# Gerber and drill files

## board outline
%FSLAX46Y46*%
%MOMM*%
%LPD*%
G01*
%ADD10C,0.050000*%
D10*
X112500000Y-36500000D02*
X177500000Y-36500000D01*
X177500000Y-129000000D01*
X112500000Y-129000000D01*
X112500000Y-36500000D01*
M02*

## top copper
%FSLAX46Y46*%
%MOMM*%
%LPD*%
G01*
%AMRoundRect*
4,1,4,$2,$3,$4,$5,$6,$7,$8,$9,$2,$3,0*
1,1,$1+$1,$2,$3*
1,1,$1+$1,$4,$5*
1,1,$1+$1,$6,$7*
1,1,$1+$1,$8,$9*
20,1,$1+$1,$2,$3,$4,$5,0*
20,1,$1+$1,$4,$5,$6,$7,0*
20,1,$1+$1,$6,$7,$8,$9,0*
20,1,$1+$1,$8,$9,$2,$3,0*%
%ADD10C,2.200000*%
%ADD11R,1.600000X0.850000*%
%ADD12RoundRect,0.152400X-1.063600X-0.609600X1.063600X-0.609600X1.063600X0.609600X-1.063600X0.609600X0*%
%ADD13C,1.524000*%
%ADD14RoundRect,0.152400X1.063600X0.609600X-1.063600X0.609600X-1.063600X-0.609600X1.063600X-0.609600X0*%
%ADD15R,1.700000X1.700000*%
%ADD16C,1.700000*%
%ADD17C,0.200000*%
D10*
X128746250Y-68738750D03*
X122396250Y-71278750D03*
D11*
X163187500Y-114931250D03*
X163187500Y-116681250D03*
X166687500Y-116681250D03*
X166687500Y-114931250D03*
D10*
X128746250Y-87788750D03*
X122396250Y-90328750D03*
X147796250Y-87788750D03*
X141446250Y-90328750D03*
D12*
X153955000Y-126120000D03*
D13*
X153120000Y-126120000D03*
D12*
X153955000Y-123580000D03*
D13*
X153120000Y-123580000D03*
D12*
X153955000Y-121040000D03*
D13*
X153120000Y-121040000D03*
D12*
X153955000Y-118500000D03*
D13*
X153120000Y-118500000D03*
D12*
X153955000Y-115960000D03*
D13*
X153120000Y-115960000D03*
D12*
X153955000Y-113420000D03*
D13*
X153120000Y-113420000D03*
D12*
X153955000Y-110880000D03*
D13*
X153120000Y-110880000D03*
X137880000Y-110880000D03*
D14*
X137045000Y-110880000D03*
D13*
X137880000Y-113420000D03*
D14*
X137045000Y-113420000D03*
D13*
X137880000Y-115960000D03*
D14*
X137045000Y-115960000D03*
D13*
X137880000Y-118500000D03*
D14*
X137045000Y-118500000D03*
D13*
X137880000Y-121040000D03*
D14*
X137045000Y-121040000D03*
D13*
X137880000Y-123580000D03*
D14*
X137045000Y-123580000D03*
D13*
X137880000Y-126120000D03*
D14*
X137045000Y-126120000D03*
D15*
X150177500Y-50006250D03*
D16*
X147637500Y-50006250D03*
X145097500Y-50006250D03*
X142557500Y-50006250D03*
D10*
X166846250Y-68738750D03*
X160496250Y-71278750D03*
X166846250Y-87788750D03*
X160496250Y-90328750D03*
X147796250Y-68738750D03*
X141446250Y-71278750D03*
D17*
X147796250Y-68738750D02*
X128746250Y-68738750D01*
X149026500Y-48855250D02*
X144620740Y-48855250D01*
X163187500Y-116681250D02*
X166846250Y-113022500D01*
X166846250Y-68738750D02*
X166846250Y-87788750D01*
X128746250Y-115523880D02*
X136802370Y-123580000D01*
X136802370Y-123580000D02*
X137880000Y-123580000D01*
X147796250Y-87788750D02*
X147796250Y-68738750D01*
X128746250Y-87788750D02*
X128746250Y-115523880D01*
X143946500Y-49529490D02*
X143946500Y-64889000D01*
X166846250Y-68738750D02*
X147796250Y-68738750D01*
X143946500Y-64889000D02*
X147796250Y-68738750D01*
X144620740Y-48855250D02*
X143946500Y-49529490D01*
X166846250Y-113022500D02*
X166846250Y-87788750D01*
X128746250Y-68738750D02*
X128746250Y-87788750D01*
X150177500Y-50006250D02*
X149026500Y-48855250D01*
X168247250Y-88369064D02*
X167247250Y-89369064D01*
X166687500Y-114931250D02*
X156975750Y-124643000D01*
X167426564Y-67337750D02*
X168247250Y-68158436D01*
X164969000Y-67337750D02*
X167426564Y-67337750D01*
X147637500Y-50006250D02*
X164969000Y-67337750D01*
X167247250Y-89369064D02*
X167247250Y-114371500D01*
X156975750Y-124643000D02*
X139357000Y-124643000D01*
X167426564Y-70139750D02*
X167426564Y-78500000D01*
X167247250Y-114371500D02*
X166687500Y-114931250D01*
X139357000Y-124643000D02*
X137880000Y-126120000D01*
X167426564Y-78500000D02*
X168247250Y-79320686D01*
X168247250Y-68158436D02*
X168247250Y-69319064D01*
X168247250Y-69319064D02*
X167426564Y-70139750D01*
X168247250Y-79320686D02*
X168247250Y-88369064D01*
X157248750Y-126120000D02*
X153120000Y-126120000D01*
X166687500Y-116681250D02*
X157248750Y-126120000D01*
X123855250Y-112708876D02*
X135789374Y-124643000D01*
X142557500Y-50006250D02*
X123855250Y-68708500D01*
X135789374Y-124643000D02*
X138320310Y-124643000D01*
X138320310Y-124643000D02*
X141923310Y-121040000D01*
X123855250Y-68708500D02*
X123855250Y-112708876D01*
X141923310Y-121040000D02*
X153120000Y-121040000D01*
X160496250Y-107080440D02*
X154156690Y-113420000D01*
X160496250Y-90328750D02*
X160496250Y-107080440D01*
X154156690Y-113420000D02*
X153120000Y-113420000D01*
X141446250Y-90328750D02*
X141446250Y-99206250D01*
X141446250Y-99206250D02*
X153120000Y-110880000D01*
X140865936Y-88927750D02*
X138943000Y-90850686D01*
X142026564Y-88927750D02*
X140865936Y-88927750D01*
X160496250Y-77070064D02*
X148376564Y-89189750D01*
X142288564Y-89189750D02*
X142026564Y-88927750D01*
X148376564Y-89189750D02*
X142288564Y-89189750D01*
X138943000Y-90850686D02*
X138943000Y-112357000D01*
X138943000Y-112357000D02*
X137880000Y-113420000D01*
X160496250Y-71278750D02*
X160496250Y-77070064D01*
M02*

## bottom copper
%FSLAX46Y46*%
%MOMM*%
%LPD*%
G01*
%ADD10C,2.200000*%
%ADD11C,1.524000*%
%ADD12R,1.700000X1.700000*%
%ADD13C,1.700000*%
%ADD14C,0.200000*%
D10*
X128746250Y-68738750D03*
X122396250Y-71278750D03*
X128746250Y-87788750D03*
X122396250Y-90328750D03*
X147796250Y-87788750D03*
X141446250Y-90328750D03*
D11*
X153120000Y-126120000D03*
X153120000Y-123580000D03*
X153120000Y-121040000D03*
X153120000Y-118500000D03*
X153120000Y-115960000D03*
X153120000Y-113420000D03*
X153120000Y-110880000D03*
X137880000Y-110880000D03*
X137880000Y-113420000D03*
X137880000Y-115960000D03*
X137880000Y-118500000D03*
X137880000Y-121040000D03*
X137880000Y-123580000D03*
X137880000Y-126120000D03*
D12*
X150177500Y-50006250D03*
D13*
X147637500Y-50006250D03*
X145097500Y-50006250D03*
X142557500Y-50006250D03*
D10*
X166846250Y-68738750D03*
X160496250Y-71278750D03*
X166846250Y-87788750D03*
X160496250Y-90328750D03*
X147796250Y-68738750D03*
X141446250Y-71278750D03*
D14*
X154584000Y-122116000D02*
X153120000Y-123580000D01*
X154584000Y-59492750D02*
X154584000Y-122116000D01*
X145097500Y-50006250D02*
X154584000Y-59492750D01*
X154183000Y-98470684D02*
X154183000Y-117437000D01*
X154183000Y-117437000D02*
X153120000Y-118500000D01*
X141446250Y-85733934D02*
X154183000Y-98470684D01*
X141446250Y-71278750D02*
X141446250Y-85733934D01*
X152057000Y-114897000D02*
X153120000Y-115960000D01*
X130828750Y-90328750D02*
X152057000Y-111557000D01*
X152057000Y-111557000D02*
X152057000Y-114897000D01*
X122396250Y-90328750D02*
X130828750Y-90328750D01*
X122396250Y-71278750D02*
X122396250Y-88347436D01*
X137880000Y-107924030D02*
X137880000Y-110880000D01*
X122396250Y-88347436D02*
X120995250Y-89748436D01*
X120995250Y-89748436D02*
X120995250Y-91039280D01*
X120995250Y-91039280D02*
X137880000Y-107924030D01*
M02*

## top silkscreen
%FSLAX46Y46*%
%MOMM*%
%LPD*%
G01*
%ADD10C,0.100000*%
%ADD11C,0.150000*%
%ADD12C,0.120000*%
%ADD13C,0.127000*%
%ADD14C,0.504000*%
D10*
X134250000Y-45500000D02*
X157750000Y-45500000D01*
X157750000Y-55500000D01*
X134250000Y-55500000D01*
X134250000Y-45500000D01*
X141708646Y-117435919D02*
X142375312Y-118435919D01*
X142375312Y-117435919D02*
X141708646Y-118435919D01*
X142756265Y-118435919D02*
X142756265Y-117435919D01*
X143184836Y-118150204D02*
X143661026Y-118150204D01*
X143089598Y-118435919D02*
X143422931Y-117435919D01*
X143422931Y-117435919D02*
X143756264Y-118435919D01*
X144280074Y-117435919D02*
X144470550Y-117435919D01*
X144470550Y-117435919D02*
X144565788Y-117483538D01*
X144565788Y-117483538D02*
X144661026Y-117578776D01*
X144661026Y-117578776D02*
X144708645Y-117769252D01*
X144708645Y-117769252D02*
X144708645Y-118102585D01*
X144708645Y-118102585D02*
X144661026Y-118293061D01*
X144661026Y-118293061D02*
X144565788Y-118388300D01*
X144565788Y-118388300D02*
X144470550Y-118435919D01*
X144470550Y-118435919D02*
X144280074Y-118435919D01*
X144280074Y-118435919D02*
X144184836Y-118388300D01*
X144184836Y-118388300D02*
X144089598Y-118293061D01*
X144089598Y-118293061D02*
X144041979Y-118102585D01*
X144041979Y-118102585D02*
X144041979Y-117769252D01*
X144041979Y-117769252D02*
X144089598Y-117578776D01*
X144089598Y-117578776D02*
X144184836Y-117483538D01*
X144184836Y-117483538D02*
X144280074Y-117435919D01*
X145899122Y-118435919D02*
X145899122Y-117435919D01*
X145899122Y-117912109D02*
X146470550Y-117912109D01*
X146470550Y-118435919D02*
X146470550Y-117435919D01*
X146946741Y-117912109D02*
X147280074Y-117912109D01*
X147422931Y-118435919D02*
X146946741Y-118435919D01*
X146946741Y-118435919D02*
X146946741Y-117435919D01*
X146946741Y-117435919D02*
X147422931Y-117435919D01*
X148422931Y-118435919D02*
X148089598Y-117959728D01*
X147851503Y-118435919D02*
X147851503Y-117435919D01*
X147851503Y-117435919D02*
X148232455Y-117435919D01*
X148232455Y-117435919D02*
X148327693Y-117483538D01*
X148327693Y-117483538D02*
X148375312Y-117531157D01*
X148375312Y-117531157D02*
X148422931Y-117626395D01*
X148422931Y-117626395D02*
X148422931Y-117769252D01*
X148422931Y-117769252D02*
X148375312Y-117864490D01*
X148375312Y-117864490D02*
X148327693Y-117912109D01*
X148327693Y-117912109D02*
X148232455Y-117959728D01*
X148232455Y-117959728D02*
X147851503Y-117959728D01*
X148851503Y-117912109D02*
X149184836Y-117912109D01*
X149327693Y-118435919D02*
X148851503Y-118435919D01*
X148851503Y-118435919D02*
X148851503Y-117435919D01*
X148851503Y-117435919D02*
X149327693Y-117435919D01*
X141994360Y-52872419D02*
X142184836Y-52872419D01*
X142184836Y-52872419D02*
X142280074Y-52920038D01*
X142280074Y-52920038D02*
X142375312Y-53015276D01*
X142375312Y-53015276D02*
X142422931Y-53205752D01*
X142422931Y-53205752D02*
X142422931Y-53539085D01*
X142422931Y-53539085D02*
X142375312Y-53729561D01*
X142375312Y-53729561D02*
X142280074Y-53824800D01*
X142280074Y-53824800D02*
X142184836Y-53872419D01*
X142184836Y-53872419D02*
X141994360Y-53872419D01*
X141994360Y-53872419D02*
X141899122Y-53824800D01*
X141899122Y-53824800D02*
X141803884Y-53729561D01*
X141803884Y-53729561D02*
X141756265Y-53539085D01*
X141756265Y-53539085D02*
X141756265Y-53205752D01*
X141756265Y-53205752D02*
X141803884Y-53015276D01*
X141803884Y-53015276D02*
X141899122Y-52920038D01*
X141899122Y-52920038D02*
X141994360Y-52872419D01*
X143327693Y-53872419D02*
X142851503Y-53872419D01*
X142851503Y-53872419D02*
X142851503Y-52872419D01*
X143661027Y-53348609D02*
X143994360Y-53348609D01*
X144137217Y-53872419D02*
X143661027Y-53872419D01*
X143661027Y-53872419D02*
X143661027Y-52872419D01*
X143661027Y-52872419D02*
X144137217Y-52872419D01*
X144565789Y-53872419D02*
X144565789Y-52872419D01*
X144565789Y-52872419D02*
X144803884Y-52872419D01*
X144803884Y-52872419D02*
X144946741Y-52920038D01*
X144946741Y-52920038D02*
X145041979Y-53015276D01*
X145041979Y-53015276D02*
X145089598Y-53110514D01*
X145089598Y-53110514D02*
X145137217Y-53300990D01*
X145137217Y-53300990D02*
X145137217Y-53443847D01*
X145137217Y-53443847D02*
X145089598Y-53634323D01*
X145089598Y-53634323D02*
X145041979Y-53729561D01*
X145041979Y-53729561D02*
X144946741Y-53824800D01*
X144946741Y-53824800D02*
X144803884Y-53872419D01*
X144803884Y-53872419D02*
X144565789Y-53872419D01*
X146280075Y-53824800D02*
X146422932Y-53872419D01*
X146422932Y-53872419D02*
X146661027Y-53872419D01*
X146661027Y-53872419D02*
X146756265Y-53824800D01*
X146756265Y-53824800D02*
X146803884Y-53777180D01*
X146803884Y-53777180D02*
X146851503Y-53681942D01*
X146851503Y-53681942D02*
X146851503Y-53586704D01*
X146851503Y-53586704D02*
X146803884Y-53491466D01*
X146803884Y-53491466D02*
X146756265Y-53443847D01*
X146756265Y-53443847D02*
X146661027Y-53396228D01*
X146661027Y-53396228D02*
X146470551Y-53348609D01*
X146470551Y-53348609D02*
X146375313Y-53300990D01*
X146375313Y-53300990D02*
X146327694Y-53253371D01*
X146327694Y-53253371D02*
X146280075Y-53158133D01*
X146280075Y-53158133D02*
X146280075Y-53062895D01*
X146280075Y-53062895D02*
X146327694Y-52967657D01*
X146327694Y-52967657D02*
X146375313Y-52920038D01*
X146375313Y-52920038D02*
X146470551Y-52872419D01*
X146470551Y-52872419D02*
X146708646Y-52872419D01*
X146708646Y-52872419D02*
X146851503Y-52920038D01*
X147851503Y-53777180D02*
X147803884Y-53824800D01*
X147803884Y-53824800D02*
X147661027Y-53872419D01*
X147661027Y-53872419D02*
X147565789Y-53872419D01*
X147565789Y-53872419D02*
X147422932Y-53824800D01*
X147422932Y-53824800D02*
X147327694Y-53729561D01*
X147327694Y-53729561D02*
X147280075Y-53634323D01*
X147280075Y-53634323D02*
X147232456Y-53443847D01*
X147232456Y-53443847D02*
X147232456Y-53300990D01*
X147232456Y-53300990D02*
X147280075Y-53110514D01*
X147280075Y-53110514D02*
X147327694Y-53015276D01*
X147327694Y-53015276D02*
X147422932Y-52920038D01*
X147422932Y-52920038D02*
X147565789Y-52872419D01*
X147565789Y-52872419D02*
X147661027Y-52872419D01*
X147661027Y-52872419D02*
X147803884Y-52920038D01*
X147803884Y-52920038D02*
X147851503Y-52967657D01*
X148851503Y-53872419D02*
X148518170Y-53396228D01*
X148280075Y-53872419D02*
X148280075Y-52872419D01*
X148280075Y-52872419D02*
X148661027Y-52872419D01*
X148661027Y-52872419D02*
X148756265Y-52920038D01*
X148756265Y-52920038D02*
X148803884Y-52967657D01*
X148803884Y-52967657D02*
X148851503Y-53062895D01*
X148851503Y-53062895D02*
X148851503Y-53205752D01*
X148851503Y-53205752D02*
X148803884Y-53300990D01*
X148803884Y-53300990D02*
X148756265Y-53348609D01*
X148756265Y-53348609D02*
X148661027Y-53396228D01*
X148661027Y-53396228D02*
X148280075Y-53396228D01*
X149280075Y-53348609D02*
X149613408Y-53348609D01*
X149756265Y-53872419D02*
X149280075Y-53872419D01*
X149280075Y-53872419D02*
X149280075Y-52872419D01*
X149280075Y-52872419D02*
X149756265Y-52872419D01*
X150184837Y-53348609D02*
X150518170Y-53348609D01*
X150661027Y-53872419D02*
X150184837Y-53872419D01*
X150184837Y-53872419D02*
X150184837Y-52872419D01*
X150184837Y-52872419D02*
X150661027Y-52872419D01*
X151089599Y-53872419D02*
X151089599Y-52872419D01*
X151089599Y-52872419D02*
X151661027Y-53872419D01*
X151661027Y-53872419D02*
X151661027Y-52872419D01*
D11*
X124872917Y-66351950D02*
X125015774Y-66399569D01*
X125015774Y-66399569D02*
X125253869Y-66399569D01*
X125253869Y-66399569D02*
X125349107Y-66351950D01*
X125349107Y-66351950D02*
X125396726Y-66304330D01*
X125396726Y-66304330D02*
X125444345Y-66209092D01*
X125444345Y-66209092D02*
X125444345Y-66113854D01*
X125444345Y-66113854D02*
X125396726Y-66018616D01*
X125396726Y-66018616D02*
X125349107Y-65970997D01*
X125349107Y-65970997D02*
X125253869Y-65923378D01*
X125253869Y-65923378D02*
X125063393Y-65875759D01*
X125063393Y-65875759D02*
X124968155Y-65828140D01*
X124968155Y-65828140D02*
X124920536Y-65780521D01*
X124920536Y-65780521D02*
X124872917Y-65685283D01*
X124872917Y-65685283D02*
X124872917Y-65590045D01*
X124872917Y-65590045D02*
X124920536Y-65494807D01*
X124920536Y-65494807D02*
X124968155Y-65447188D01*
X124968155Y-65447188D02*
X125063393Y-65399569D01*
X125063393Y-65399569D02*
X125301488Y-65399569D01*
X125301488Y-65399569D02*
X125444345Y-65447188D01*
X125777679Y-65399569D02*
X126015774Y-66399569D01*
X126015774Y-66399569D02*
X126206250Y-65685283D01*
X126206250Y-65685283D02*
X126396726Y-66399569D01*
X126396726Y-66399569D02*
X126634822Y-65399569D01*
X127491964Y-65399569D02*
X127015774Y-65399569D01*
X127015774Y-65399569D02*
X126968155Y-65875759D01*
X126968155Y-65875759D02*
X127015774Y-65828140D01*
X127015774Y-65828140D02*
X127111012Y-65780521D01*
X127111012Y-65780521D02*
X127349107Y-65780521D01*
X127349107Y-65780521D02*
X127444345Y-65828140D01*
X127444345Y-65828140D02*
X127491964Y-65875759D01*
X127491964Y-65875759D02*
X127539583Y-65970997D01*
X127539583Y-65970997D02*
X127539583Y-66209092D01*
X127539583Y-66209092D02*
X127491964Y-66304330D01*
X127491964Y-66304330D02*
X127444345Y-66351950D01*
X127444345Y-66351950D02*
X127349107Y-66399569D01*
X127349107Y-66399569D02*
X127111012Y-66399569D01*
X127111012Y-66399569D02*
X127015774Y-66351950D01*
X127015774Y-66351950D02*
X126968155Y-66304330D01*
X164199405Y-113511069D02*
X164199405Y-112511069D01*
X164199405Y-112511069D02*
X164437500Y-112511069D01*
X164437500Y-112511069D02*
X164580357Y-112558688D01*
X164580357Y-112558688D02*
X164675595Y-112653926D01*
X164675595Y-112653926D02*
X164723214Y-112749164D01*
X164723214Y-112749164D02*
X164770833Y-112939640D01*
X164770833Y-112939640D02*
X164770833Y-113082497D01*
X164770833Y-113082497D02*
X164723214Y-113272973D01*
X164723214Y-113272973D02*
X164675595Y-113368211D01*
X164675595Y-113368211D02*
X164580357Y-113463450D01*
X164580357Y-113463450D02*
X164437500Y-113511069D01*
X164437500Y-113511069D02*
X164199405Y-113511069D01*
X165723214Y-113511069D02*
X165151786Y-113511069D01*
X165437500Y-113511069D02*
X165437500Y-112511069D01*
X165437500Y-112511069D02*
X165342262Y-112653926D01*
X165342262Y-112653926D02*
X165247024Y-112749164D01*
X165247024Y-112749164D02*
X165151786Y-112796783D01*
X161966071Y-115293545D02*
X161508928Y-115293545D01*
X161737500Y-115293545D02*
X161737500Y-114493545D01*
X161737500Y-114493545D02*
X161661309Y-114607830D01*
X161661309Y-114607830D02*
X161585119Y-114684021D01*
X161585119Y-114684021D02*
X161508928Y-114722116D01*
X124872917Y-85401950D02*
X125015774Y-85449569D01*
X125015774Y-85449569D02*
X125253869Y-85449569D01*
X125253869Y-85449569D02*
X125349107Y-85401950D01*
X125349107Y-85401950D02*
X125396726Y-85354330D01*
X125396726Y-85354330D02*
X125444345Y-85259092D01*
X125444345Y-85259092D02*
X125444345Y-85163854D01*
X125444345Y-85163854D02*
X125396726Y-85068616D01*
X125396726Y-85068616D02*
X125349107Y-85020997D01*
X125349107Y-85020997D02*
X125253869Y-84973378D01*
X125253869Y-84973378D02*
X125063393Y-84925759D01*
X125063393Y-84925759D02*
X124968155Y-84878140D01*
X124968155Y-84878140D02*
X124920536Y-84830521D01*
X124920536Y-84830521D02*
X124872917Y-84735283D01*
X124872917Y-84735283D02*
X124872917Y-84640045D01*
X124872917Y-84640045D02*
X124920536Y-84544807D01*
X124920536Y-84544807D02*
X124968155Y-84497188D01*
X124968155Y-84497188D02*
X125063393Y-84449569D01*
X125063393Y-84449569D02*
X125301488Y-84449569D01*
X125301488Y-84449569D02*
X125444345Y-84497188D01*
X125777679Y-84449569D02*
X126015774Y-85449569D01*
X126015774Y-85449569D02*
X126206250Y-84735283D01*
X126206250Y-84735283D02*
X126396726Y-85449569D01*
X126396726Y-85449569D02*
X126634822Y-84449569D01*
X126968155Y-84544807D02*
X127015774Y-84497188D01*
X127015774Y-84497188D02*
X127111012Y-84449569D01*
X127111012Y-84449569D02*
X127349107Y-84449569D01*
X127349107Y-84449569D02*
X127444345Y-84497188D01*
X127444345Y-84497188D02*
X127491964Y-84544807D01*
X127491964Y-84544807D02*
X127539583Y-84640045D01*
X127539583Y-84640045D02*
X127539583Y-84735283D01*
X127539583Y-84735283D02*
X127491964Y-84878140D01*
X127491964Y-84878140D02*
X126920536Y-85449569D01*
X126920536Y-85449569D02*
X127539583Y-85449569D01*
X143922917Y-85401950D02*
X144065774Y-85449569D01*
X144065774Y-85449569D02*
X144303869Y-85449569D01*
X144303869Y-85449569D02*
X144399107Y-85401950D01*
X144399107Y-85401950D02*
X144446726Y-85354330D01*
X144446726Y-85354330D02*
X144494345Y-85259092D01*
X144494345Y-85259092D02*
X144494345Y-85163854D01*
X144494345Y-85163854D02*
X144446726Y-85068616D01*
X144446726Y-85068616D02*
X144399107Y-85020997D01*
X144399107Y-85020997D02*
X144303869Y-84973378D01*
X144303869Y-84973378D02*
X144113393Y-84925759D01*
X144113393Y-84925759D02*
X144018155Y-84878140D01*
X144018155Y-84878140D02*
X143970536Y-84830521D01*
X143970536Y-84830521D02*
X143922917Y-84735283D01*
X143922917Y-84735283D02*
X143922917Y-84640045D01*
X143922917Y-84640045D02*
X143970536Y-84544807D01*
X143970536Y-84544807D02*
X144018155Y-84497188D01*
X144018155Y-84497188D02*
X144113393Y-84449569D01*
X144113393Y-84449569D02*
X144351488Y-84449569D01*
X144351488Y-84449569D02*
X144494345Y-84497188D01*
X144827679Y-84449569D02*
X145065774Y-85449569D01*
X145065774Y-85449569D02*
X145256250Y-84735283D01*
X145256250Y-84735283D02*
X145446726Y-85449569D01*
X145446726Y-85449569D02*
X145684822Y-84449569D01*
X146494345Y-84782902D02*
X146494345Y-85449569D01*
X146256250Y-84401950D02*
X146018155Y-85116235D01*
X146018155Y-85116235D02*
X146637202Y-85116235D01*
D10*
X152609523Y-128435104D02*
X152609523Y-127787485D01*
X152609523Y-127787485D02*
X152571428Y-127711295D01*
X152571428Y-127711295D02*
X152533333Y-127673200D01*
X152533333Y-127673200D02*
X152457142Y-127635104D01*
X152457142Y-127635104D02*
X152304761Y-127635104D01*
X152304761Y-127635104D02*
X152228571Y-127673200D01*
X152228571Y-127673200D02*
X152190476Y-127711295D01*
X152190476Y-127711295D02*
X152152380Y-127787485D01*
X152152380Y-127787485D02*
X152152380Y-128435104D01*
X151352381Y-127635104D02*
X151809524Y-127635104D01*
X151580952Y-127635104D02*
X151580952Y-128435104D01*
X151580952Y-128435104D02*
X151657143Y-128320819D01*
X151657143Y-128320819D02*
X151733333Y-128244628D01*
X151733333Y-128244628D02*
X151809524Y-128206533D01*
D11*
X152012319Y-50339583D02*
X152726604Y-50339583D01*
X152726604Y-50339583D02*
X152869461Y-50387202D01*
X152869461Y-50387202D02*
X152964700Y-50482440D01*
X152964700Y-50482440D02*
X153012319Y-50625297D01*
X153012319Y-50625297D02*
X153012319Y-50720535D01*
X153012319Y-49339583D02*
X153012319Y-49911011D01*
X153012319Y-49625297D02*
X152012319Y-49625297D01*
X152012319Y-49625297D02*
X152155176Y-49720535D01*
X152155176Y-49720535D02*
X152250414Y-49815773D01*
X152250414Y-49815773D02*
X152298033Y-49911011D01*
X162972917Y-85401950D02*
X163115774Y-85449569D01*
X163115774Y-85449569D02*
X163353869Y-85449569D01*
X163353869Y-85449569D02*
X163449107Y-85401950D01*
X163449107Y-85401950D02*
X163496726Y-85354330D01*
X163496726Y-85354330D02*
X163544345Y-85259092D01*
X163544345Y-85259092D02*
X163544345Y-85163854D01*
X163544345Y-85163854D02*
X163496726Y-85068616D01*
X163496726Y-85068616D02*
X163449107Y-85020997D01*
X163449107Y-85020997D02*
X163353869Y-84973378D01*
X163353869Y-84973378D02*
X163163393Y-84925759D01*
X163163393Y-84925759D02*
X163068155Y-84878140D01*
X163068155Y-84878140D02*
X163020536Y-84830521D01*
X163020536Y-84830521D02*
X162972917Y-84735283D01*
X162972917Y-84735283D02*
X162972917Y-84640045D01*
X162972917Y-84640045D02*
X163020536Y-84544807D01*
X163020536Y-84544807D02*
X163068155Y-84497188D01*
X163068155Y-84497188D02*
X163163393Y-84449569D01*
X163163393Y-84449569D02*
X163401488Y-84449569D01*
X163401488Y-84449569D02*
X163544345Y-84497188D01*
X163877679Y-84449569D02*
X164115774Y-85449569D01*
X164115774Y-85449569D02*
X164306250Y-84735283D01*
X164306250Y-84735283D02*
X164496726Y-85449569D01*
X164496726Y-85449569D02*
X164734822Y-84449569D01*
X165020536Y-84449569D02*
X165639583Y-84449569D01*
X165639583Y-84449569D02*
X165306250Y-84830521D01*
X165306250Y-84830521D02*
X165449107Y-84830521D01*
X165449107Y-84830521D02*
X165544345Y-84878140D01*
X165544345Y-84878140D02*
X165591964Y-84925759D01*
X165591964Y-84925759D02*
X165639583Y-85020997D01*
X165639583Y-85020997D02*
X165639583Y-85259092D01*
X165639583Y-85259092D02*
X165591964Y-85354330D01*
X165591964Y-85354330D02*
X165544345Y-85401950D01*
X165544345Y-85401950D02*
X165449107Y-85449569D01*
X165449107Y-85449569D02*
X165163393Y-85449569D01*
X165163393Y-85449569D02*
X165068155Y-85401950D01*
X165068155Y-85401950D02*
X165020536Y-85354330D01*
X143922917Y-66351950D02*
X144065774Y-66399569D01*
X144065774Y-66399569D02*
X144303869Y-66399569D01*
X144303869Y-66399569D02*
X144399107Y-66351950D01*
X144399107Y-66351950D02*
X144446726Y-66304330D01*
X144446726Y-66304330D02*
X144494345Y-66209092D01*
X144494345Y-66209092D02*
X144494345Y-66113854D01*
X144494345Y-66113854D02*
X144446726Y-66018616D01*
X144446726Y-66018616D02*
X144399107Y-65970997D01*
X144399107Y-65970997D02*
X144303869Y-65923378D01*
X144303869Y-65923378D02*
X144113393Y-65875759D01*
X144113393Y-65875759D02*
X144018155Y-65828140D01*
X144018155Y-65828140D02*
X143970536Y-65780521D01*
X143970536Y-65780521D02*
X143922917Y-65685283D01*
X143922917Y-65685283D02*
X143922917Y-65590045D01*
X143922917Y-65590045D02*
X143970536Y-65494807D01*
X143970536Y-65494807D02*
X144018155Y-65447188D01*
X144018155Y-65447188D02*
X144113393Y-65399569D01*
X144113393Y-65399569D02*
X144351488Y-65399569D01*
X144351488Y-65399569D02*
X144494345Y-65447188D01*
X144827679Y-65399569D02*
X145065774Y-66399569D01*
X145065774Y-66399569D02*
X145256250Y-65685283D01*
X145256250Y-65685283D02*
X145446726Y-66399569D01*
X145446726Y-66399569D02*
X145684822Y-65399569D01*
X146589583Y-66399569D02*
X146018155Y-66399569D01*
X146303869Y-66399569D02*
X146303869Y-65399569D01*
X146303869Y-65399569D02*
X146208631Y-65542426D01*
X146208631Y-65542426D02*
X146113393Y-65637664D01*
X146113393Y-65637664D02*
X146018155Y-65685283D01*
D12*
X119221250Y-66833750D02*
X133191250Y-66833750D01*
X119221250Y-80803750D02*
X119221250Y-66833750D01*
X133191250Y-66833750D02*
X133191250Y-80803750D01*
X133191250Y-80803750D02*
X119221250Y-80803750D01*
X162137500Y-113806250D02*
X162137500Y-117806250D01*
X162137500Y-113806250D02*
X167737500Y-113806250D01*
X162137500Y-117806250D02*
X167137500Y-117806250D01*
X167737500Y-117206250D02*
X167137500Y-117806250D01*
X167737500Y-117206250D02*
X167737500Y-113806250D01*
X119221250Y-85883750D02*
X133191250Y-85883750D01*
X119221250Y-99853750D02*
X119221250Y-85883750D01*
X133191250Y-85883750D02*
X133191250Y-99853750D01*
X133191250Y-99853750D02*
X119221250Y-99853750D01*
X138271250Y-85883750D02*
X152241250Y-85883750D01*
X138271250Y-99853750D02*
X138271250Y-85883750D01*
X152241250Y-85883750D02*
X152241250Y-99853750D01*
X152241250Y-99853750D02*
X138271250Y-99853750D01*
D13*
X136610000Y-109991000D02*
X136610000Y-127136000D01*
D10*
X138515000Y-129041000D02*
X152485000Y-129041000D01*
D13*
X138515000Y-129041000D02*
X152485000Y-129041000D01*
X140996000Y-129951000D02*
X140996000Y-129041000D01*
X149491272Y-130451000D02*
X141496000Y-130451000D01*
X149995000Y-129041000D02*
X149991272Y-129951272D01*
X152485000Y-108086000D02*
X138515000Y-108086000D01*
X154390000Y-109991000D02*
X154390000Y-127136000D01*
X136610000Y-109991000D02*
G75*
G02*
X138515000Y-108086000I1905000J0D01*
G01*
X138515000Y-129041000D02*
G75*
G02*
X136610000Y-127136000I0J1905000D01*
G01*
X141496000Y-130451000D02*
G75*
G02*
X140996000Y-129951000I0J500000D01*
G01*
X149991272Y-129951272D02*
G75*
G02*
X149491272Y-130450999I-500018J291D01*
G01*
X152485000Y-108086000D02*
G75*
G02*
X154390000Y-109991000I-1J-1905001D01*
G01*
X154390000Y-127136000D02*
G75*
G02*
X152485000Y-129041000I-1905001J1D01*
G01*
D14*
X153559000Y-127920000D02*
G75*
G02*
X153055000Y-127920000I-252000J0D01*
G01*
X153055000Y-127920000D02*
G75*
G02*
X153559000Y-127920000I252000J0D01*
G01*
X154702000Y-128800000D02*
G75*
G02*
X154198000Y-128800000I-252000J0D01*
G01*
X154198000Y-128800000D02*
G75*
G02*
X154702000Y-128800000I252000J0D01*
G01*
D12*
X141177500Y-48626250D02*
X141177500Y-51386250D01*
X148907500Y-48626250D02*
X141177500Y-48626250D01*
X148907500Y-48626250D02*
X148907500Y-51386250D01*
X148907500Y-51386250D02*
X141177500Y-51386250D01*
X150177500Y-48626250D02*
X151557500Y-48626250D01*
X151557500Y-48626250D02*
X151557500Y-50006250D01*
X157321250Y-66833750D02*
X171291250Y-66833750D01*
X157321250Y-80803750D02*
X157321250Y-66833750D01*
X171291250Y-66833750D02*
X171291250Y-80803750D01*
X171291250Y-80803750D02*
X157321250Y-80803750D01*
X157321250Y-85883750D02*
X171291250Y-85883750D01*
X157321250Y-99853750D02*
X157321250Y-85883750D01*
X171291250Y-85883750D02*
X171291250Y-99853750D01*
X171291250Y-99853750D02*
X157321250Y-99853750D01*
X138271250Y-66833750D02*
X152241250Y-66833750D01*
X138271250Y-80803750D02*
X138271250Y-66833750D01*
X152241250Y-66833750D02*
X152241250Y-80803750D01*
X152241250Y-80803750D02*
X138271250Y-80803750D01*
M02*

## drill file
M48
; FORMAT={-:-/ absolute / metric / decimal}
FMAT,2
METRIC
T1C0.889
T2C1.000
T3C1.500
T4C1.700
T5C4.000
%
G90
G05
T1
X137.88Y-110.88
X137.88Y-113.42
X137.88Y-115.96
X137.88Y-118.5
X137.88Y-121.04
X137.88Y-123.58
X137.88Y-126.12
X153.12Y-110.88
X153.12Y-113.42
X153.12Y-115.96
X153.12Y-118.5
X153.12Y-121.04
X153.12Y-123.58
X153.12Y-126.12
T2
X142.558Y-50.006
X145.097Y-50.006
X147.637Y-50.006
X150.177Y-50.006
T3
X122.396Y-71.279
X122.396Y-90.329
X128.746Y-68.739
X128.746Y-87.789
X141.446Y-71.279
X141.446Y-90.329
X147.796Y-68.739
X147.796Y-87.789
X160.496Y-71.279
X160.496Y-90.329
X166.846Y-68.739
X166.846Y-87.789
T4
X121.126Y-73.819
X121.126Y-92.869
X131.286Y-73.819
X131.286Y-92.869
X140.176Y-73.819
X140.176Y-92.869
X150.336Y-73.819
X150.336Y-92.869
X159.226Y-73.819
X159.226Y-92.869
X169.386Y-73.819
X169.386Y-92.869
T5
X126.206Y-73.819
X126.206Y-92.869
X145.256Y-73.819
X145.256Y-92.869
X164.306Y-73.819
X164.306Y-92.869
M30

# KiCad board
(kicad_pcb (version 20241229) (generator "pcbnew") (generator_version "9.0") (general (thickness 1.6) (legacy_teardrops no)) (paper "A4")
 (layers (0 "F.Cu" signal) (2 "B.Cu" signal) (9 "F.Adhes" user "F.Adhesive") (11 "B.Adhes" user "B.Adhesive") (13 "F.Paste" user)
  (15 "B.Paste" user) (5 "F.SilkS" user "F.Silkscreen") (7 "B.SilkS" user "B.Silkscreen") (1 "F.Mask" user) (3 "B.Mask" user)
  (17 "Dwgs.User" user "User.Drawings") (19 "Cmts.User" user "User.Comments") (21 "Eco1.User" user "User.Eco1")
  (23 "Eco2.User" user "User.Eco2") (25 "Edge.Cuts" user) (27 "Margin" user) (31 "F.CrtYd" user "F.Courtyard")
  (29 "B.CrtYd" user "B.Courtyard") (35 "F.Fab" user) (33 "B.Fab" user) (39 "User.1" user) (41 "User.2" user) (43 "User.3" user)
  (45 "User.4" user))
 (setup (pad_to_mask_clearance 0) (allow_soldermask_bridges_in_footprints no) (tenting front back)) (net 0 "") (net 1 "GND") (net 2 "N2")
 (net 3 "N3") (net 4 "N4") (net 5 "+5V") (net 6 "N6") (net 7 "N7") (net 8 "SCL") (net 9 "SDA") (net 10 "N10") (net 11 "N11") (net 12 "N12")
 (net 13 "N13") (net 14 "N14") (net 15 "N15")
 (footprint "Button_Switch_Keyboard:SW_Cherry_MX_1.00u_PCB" (layer "F.Cu") (at 128.74625 68.73875)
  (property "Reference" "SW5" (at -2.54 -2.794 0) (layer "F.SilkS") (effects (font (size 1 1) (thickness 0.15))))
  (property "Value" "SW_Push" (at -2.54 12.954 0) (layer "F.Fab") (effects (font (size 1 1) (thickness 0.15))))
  (fp_line (start -9.525 -1.905) (end 4.445 -1.905) (stroke (width 0.12) (type solid)) (layer "F.SilkS"))
  (fp_line (start -9.525 12.065) (end -9.525 -1.905) (stroke (width 0.12) (type solid)) (layer "F.SilkS"))
  (fp_line (start 4.445 -1.905) (end 4.445 12.065) (stroke (width 0.12) (type solid)) (layer "F.SilkS"))
  (fp_line (start 4.445 12.065) (end -9.525 12.065) (stroke (width 0.12) (type solid)) (layer "F.SilkS"))
  (pad "" np_thru_hole circle (at -7.62 5.08) (size 1.7 1.7) (drill 1.7) (layers "*.Cu" "*.Mask"))
  (pad "" np_thru_hole circle (at -2.54 5.08) (size 4 4) (drill 4) (layers "*.Cu" "*.Mask"))
  (pad "" np_thru_hole circle (at 2.54 5.08) (size 1.7 1.7) (drill 1.7) (layers "*.Cu" "*.Mask"))
  (pad "1" thru_hole circle (at 0 0) (size 2.2 2.2) (drill 1.5) (layers "*.Cu" "*.Mask") (remove_unused_layers no) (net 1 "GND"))
  (pad "2" thru_hole circle (at -6.35 2.54) (size 2.2 2.2) (drill 1.5) (layers "*.Cu" "*.Mask") (remove_unused_layers no) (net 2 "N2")))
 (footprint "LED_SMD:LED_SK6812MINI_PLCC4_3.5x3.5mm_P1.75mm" (layer "F.Cu") (at 164.9375 115.80625)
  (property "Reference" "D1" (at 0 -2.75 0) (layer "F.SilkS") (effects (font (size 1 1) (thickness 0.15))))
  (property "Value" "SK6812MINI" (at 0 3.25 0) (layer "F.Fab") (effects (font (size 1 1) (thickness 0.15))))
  (fp_line (start -2.8 -2) (end -2.8 2) (stroke (width 0.12) (type default)) (layer "F.SilkS"))
  (fp_line (start -2.8 -2) (end 2.8 -2) (stroke (width 0.12) (type solid)) (layer "F.SilkS"))
  (fp_line (start -2.8 2) (end 2.2 2) (stroke (width 0.12) (type solid)) (layer "F.SilkS"))
  (fp_line (start 2.8 1.4) (end 2.2 2) (stroke (width 0.12) (type default)) (layer "F.SilkS"))
  (fp_line (start 2.8 1.4) (end 2.8 -2) (stroke (width 0.12) (type solid)) (layer "F.SilkS"))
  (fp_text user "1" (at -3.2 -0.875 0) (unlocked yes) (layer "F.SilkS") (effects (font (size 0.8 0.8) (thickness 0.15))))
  (pad "1" smd rect (at -1.75 -0.875) (size 1.6 0.85) (layers "F.Cu" "F.Mask" "F.Paste") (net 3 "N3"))
  (pad "2" smd rect (at -1.75 0.875) (size 1.6 0.85) (layers "F.Cu" "F.Mask" "F.Paste") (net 1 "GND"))
  (pad "3" smd rect (at 1.75 0.875) (size 1.6 0.85) (layers "F.Cu" "F.Mask" "F.Paste") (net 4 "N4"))
  (pad "4" smd rect (at 1.75 -0.875) (size 1.6 0.85) (layers "F.Cu" "F.Mask" "F.Paste") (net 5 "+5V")))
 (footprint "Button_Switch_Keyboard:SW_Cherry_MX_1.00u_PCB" (layer "F.Cu") (at 128.74625 87.78875)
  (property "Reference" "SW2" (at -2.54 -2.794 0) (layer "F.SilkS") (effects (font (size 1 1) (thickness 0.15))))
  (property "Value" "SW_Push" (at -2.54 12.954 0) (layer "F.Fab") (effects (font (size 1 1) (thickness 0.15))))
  (fp_line (start -9.525 -1.905) (end 4.445 -1.905) (stroke (width 0.12) (type solid)) (layer "F.SilkS"))
  (fp_line (start -9.525 12.065) (end -9.525 -1.905) (stroke (width 0.12) (type solid)) (layer "F.SilkS"))
  (fp_line (start 4.445 -1.905) (end 4.445 12.065) (stroke (width 0.12) (type solid)) (layer "F.SilkS"))
  (fp_line (start 4.445 12.065) (end -9.525 12.065) (stroke (width 0.12) (type solid)) (layer "F.SilkS"))
  (pad "" np_thru_hole circle (at -7.62 5.08) (size 1.7 1.7) (drill 1.7) (layers "*.Cu" "*.Mask"))
  (pad "" np_thru_hole circle (at -2.54 5.08) (size 4 4) (drill 4) (layers "*.Cu" "*.Mask"))
  (pad "" np_thru_hole circle (at 2.54 5.08) (size 1.7 1.7) (drill 1.7) (layers "*.Cu" "*.Mask"))
  (pad "1" thru_hole circle (at 0 0) (size 2.2 2.2) (drill 1.5) (layers "*.Cu" "*.Mask") (remove_unused_layers no) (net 1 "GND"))
  (pad "2" thru_hole circle (at -6.35 2.54) (size 2.2 2.2) (drill 1.5) (layers "*.Cu" "*.Mask") (remove_unused_layers no) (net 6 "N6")))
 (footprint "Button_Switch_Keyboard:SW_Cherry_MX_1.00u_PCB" (layer "F.Cu") (at 147.79625 87.78875)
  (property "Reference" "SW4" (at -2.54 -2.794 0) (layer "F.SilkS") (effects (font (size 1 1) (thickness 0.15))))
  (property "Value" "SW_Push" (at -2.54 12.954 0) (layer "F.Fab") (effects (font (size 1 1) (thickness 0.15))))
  (fp_line (start -9.525 -1.905) (end 4.445 -1.905) (stroke (width 0.12) (type solid)) (layer "F.SilkS"))
  (fp_line (start -9.525 12.065) (end -9.525 -1.905) (stroke (width 0.12) (type solid)) (layer "F.SilkS"))
  (fp_line (start 4.445 -1.905) (end 4.445 12.065) (stroke (width 0.12) (type solid)) (layer "F.SilkS"))
  (fp_line (start 4.445 12.065) (end -9.525 12.065) (stroke (width 0.12) (type solid)) (layer "F.SilkS"))
  (pad "" np_thru_hole circle (at -7.62 5.08) (size 1.7 1.7) (drill 1.7) (layers "*.Cu" "*.Mask"))
  (pad "" np_thru_hole circle (at -2.54 5.08) (size 4 4) (drill 4) (layers "*.Cu" "*.Mask"))
  (pad "" np_thru_hole circle (at 2.54 5.08) (size 1.7 1.7) (drill 1.7) (layers "*.Cu" "*.Mask"))
  (pad "1" thru_hole circle (at 0 0) (size 2.2 2.2) (drill 1.5) (layers "*.Cu" "*.Mask") (remove_unused_layers no) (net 1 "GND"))
  (pad "2" thru_hole circle (at -6.35 2.54) (size 2.2 2.2) (drill 1.5) (layers "*.Cu" "*.Mask") (remove_unused_layers no) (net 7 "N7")))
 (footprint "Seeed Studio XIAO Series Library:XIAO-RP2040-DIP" (layer "F.Cu") (at 145.5 118.5 180)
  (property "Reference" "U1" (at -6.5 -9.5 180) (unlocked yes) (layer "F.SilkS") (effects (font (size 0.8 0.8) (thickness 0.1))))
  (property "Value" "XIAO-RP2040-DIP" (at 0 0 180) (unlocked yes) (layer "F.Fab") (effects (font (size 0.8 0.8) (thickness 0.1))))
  (fp_line (start 8.89 8.509) (end 8.89 -8.636) (stroke (width 0.127) (type solid)) (layer "F.SilkS"))
  (fp_line (start 6.985 -10.541) (end -6.985 -10.541) (stroke (width 0.1) (type solid)) (layer "F.SilkS"))
  (fp_line (start 6.985 -10.541) (end -6.985 -10.541) (stroke (width 0.127) (type solid)) (layer "F.SilkS"))
  (fp_line (start 4.504 -11.451) (end 4.504 -10.541) (stroke (width 0.127) (type solid)) (layer "F.SilkS"))
  (fp_line (start -3.991272 -11.951) (end 4.004 -11.951) (stroke (width 0.127) (type solid)) (layer "F.SilkS"))
  (fp_line (start -4.495 -10.541) (end -4.491272 -11.451272) (stroke (width 0.127) (type solid)) (layer "F.SilkS"))
  (fp_line (start -6.985 10.414) (end 6.985 10.414) (stroke (width 0.127) (type solid)) (layer "F.SilkS"))
  (fp_line (start -8.89 8.509) (end -8.89 -8.636) (stroke (width 0.127) (type solid)) (layer "F.SilkS"))
  (fp_arc (start 8.89 8.509) (mid 8.332038 9.856038) (end 6.985 10.414) (stroke (width 0.127) (type solid)) (layer "F.SilkS"))
  (fp_arc (start 6.985 -10.541) (mid 8.332038 -9.983038) (end 8.89 -8.636) (stroke (width 0.127) (type solid)) (layer "F.SilkS"))
  (fp_arc (start 4.004 -11.951) (mid 4.357553 -11.804553) (end 4.504 -11.451) (stroke (width 0.127) (type default)) (layer "F.SilkS"))
  (fp_arc (start -4.491272 -11.451272) (mid -4.344728 -11.80464) (end -3.991272 -11.951) (stroke (width 0.127) (type default))
   (layer "F.SilkS"))
  (fp_arc (start -6.985 10.414) (mid -8.332038 9.856038) (end -8.89 8.509) (stroke (width 0.127) (type solid)) (layer "F.SilkS"))
  (fp_arc (start -8.89 -8.636) (mid -8.332038 -9.983038) (end -6.985 -10.541) (stroke (width 0.127) (type solid)) (layer "F.SilkS"))
  (fp_circle (center -7.807 -9.42) (end -7.807 -9.674) (stroke (width 0.5) (type solid)) (fill yes) (layer "F.SilkS"))
  (fp_circle (center -8.95 -10.3) (end -8.95 -10.554) (stroke (width 0.5) (type solid)) (fill yes) (layer "F.SilkS"))
  (pad "1" smd roundrect (at -8.455 -7.62) (size 2.432 1.524) (layers "F.Cu" "F.Mask") (roundrect_rratio 0.1) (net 4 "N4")
   (thermal_bridge_angle 45))
  (pad "1" thru_hole circle (at -7.62 -7.62) (size 1.524 1.524) (drill 0.889) (layers "*.Cu" "*.Mask") (remove_unused_layers no)
   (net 4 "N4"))
  (pad "2" smd roundrect (at -8.455 -5.08) (size 2.432 1.524) (layers "F.Cu" "F.Mask") (roundrect_rratio 0.1) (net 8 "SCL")
   (thermal_bridge_angle 45))
  (pad "2" thru_hole circle (at -7.62 -5.08) (size 1.524 1.524) (drill 0.889) (layers "*.Cu" "*.Mask") (remove_unused_layers no)
   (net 8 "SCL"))
  (pad "3" smd roundrect (at -8.455 -2.54) (size 2.432 1.524) (layers "F.Cu" "F.Mask") (roundrect_rratio 0.1) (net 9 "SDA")
   (thermal_bridge_angle 45))
  (pad "3" thru_hole circle (at -7.62 -2.54) (size 1.524 1.524) (drill 0.889) (layers "*.Cu" "*.Mask") (remove_unused_layers no)
   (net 9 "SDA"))
  (pad "4" smd roundrect (at -8.455 0) (size 2.432 1.524) (layers "F.Cu" "F.Mask") (roundrect_rratio 0.1) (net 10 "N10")
   (thermal_bridge_angle 45))
  (pad "4" thru_hole circle (at -7.62 0) (size 1.524 1.524) (drill 0.889) (layers "*.Cu" "*.Mask") (remove_unused_layers no) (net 10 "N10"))
  (pad "5" smd roundrect (at -8.455 2.54) (size 2.432 1.524) (layers "F.Cu" "F.Mask") (roundrect_rratio 0.1) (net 6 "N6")
   (thermal_bridge_angle 45))
  (pad "5" thru_hole circle (at -7.62 2.54) (size 1.524 1.524) (drill 0.889) (layers "*.Cu" "*.Mask") (remove_unused_layers no) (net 6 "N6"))
  (pad "6" smd roundrect (at -8.455 5.08) (size 2.432 1.524) (layers "F.Cu" "F.Mask") (roundrect_rratio 0.1) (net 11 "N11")
   (thermal_bridge_angle 45))
  (pad "6" thru_hole circle (at -7.62 5.08) (size 1.524 1.524) (drill 0.889) (layers "*.Cu" "*.Mask") (remove_unused_layers no)
   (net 11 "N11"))
  (pad "7" smd roundrect (at -8.455 7.62) (size 2.432 1.524) (layers "F.Cu" "F.Mask") (roundrect_rratio 0.1) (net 7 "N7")
   (thermal_bridge_angle 45))
  (pad "7" thru_hole circle (at -7.62 7.62) (size 1.524 1.524) (drill 0.889) (layers "*.Cu" "*.Mask") (remove_unused_layers no) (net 7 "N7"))
  (pad "8" thru_hole circle (at 7.62 7.62 180) (size 1.524 1.524) (drill 0.889) (layers "*.Cu" "*.Mask") (remove_unused_layers no)
   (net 2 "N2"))
  (pad "8" smd roundrect (at 8.455 7.62 180) (size 2.432 1.524) (layers "F.Cu" "F.Mask") (roundrect_rratio 0.1) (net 2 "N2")
   (thermal_bridge_angle 45))
  (pad "9" thru_hole circle (at 7.62 5.08 180) (size 1.524 1.524) (drill 0.889) (layers "*.Cu" "*.Mask") (remove_unused_layers no)
   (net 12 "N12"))
  (pad "9" smd roundrect (at 8.455 5.08 180) (size 2.432 1.524) (layers "F.Cu" "F.Mask") (roundrect_rratio 0.1) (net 12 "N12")
   (thermal_bridge_angle 45))
  (pad "10" thru_hole circle (at 7.62 2.54 180) (size 1.524 1.524) (drill 0.889) (layers "*.Cu" "*.Mask") (remove_unused_layers no)
   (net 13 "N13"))
  (pad "10" smd roundrect (at 8.455 2.54 180) (size 2.432 1.524) (layers "F.Cu" "F.Mask") (roundrect_rratio 0.1) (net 13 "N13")
   (thermal_bridge_angle 45))
  (pad "11" thru_hole circle (at 7.62 0 180) (size 1.524 1.524) (drill 0.889) (layers "*.Cu" "*.Mask") (remove_unused_layers no)
   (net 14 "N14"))
  (pad "11" smd roundrect (at 8.455 0 180) (size 2.432 1.524) (layers "F.Cu" "F.Mask") (roundrect_rratio 0.1) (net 14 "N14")
   (thermal_bridge_angle 45))
  (pad "12" thru_hole circle (at 7.62 -2.54 180) (size 1.524 1.524) (drill 0.889) (layers "*.Cu" "*.Mask") (remove_unused_layers no)
   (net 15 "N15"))
  (pad "12" smd roundrect (at 8.455 -2.54 180) (size 2.432 1.524) (layers "F.Cu" "F.Mask") (roundrect_rratio 0.1) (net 15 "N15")
   (thermal_bridge_angle 45))
  (pad "13" thru_hole circle (at 7.62 -5.08 180) (size 1.524 1.524) (drill 0.889) (layers "*.Cu" "*.Mask") (remove_unused_layers no)
   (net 1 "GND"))
  (pad "13" smd roundrect (at 8.455 -5.08 180) (size 2.432 1.524) (layers "F.Cu" "F.Mask") (roundrect_rratio 0.1) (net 1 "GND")
   (thermal_bridge_angle 45))
  (pad "14" thru_hole circle (at 7.62 -7.62 180) (size 1.524 1.524) (drill 0.889) (layers "*.Cu" "*.Mask") (remove_unused_layers no)
   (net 5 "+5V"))
  (pad "14" smd roundrect (at 8.455 -7.62 180) (size 2.432 1.524) (layers "F.Cu" "F.Mask") (roundrect_rratio 0.1) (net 5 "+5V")
   (thermal_bridge_angle 45)))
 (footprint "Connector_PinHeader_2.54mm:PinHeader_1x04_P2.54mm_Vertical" (layer "F.Cu") (at 150.1775 50.00625 -90)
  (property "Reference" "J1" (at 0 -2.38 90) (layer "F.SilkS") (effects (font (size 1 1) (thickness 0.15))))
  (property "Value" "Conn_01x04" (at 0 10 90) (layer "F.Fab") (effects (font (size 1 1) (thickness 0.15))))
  (fp_line (start -1.38 9) (end 1.38 9) (stroke (width 0.12) (type solid)) (layer "F.SilkS"))
  (fp_line (start -1.38 1.27) (end -1.38 9) (stroke (width 0.12) (type solid)) (layer "F.SilkS"))
  (fp_line (start -1.38 1.27) (end 1.38 1.27) (stroke (width 0.12) (type solid)) (layer "F.SilkS"))
  (fp_line (start 1.38 1.27) (end 1.38 9) (stroke (width 0.12) (type solid)) (layer "F.SilkS"))
  (fp_line (start -1.38 0) (end -1.38 -1.38) (stroke (width 0.12) (type solid)) (layer "F.SilkS"))
  (fp_line (start -1.38 -1.38) (end 0 -1.38) (stroke (width 0.12) (type solid)) (layer "F.SilkS"))
  (pad "1" thru_hole rect (at 0 0 270) (size 1.7 1.7) (drill 1) (layers "*.Cu" "*.Mask") (remove_unused_layers no) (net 1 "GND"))
  (pad "2" thru_hole circle (at 0 2.54 270) (size 1.7 1.7) (drill 1) (layers "*.Cu" "*.Mask") (remove_unused_layers no) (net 5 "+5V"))
  (pad "3" thru_hole circle (at 0 5.08 270) (size 1.7 1.7) (drill 1) (layers "*.Cu" "*.Mask") (remove_unused_layers no) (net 8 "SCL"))
  (pad "4" thru_hole circle (at 0 7.62 270) (size 1.7 1.7) (drill 1) (layers "*.Cu" "*.Mask") (remove_unused_layers no) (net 9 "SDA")))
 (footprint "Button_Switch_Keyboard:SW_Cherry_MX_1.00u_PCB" (layer "F.Cu") (at 166.84625 68.73875)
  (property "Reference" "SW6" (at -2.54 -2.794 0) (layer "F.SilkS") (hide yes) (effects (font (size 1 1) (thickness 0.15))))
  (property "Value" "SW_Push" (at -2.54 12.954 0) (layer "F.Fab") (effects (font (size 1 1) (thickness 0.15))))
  (fp_line (start -9.525 -1.905) (end 4.445 -1.905) (stroke (width 0.12) (type solid)) (layer "F.SilkS"))
  (fp_line (start -9.525 12.065) (end -9.525 -1.905) (stroke (width 0.12) (type solid)) (layer "F.SilkS"))
  (fp_line (start 4.445 -1.905) (end 4.445 12.065) (stroke (width 0.12) (type solid)) (layer "F.SilkS"))
  (fp_line (start 4.445 12.065) (end -9.525 12.065) (stroke (width 0.12) (type solid)) (layer "F.SilkS"))
  (pad "" np_thru_hole circle (at -7.62 5.08) (size 1.7 1.7) (drill 1.7) (layers "*.Cu" "*.Mask"))
  (pad "" np_thru_hole circle (at -2.54 5.08) (size 4 4) (drill 4) (layers "*.Cu" "*.Mask"))
  (pad "" np_thru_hole circle (at 2.54 5.08) (size 1.7 1.7) (drill 1.7) (layers "*.Cu" "*.Mask"))
  (pad "1" thru_hole circle (at 0 0) (size 2.2 2.2) (drill 1.5) (layers "*.Cu" "*.Mask") (remove_unused_layers no) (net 1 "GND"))
  (pad "2" thru_hole circle (at -6.35 2.54) (size 2.2 2.2) (drill 1.5) (layers "*.Cu" "*.Mask") (remove_unused_layers no) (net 12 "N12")))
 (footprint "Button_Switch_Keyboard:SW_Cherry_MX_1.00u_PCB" (layer "F.Cu") (at 166.84625 87.78875)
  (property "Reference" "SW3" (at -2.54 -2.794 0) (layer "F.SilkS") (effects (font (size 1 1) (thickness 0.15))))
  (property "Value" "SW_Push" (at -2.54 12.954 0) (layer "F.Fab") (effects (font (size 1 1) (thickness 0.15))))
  (fp_line (start -9.525 -1.905) (end 4.445 -1.905) (stroke (width 0.12) (type solid)) (layer "F.SilkS"))
  (fp_line (start -9.525 12.065) (end -9.525 -1.905) (stroke (width 0.12) (type solid)) (layer "F.SilkS"))
  (fp_line (start 4.445 -1.905) (end 4.445 12.065) (stroke (width 0.12) (type solid)) (layer "F.SilkS"))
  (fp_line (start 4.445 12.065) (end -9.525 12.065) (stroke (width 0.12) (type solid)) (layer "F.SilkS"))
  (pad "" np_thru_hole circle (at -7.62 5.08) (size 1.7 1.7) (drill 1.7) (layers "*.Cu" "*.Mask"))
  (pad "" np_thru_hole circle (at -2.54 5.08) (size 4 4) (drill 4) (layers "*.Cu" "*.Mask"))
  (pad "" np_thru_hole circle (at 2.54 5.08) (size 1.7 1.7) (drill 1.7) (layers "*.Cu" "*.Mask"))
  (pad "1" thru_hole circle (at 0 0) (size 2.2 2.2) (drill 1.5) (layers "*.Cu" "*.Mask") (remove_unused_layers no) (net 1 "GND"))
  (pad "2" thru_hole circle (at -6.35 2.54) (size 2.2 2.2) (drill 1.5) (layers "*.Cu" "*.Mask") (remove_unused_layers no) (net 11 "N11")))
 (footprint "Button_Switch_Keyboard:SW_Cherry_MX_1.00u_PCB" (layer "F.Cu") (at 147.79625 68.73875)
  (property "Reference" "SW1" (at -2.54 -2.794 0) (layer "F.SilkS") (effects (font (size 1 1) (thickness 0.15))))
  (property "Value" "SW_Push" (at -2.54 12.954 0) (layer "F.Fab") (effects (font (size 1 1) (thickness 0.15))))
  (fp_line (start -9.525 -1.905) (end 4.445 -1.905) (stroke (width 0.12) (type solid)) (layer "F.SilkS"))
  (fp_line (start -9.525 12.065) (end -9.525 -1.905) (stroke (width 0.12) (type solid)) (layer "F.SilkS"))
  (fp_line (start 4.445 -1.905) (end 4.445 12.065) (stroke (width 0.12) (type solid)) (layer "F.SilkS"))
  (fp_line (start 4.445 12.065) (end -9.525 12.065) (stroke (width 0.12) (type solid)) (layer "F.SilkS"))
  (pad "" np_thru_hole circle (at -7.62 5.08) (size 1.7 1.7) (drill 1.7) (layers "*.Cu" "*.Mask"))
  (pad "" np_thru_hole circle (at -2.54 5.08) (size 4 4) (drill 4) (layers "*.Cu" "*.Mask"))
  (pad "" np_thru_hole circle (at 2.54 5.08) (size 1.7 1.7) (drill 1.7) (layers "*.Cu" "*.Mask"))
  (pad "1" thru_hole circle (at 0 0) (size 2.2 2.2) (drill 1.5) (layers "*.Cu" "*.Mask") (remove_unused_layers no) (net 1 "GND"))
  (pad "2" thru_hole circle (at -6.35 2.54) (size 2.2 2.2) (drill 1.5) (layers "*.Cu" "*.Mask") (remove_unused_layers no) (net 10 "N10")))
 (gr_rect (start 134.25 45.5) (end 157.75 55.5) (stroke (width 0.1) (type default)) (fill no) (layer "F.SilkS"))
 (gr_rect (start 112.5 36.5) (end 177.5 129) (stroke (width 0.05) (type default)) (fill no) (layer "Edge.Cuts"))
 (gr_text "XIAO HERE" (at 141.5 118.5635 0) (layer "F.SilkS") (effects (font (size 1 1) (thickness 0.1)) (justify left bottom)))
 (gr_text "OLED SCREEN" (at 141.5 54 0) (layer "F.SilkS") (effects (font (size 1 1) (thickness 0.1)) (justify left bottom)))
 (segment (start 147.79625 68.73875) (end 128.74625 68.73875) (width 0.2) (layer "F.Cu") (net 1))
 (segment (start 149.0265 48.85525) (end 144.62074 48.85525) (width 0.2) (layer "F.Cu") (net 1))
 (segment (start 163.1875 116.68125) (end 166.84625 113.0225) (width 0.2) (layer "F.Cu") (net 1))
 (segment (start 166.84625 68.73875) (end 166.84625 87.78875) (width 0.2) (layer "F.Cu") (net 1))
 (segment (start 128.74625 115.52388) (end 136.80237 123.58) (width 0.2) (layer "F.Cu") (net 1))
 (segment (start 136.80237 123.58) (end 137.88 123.58) (width 0.2) (layer "F.Cu") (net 1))
 (segment (start 147.79625 87.78875) (end 147.79625 68.73875) (width 0.2) (layer "F.Cu") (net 1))
 (segment (start 128.74625 87.78875) (end 128.74625 115.52388) (width 0.2) (layer "F.Cu") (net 1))
 (segment (start 143.9465 49.52949) (end 143.9465 64.889) (width 0.2) (layer "F.Cu") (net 1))
 (segment (start 166.84625 68.73875) (end 147.79625 68.73875) (width 0.2) (layer "F.Cu") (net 1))
 (segment (start 143.9465 64.889) (end 147.79625 68.73875) (width 0.2) (layer "F.Cu") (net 1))
 (segment (start 144.62074 48.85525) (end 143.9465 49.52949) (width 0.2) (layer "F.Cu") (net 1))
 (segment (start 166.84625 113.0225) (end 166.84625 87.78875) (width 0.2) (layer "F.Cu") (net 1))
 (segment (start 128.74625 68.73875) (end 128.74625 87.78875) (width 0.2) (layer "F.Cu") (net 1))
 (segment (start 150.1775 50.00625) (end 149.0265 48.85525) (width 0.2) (layer "F.Cu") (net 1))
 (segment (start 168.24725 88.369064) (end 167.24725 89.369064) (width 0.2) (layer "F.Cu") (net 5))
 (segment (start 166.6875 114.93125) (end 156.97575 124.643) (width 0.2) (layer "F.Cu") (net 5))
 (segment (start 167.426564 67.33775) (end 168.24725 68.158436) (width 0.2) (layer "F.Cu") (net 5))
 (segment (start 164.969 67.33775) (end 167.426564 67.33775) (width 0.2) (layer "F.Cu") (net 5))
 (segment (start 147.6375 50.00625) (end 164.969 67.33775) (width 0.2) (layer "F.Cu") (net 5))
 (segment (start 167.24725 89.369064) (end 167.24725 114.3715) (width 0.2) (layer "F.Cu") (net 5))
 (segment (start 156.97575 124.643) (end 139.357 124.643) (width 0.2) (layer "F.Cu") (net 5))
 (segment (start 167.426564 70.13975) (end 167.426564 78.5) (width 0.2) (layer "F.Cu") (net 5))
 (segment (start 167.24725 114.3715) (end 166.6875 114.93125) (width 0.2) (layer "F.Cu") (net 5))
 (segment (start 139.357 124.643) (end 137.88 126.12) (width 0.2) (layer "F.Cu") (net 5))
 (segment (start 167.426564 78.5) (end 168.24725 79.320686) (width 0.2) (layer "F.Cu") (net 5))
 (segment (start 168.24725 68.158436) (end 168.24725 69.319064) (width 0.2) (layer "F.Cu") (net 5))
 (segment (start 168.24725 69.319064) (end 167.426564 70.13975) (width 0.2) (layer "F.Cu") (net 5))
 (segment (start 168.24725 79.320686) (end 168.24725 88.369064) (width 0.2) (layer "F.Cu") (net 5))
 (segment (start 157.24875 126.12) (end 153.12 126.12) (width 0.2) (layer "F.Cu") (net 4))
 (segment (start 166.6875 116.68125) (end 157.24875 126.12) (width 0.2) (layer "F.Cu") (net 4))
 (segment (start 154.584 122.116) (end 153.12 123.58) (width 0.2) (layer "B.Cu") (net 8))
 (segment (start 154.584 59.49275) (end 154.584 122.116) (width 0.2) (layer "B.Cu") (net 8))
 (segment (start 145.0975 50.00625) (end 154.584 59.49275) (width 0.2) (layer "B.Cu") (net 8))
 (segment (start 123.85525 112.708876) (end 135.789374 124.643) (width 0.2) (layer "F.Cu") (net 9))
 (segment (start 142.5575 50.00625) (end 123.85525 68.7085) (width 0.2) (layer "F.Cu") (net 9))
 (segment (start 135.789374 124.643) (end 138.32031 124.643) (width 0.2) (layer "F.Cu") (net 9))
 (segment (start 138.32031 124.643) (end 141.92331 121.04) (width 0.2) (layer "F.Cu") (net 9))
 (segment (start 123.85525 68.7085) (end 123.85525 112.708876) (width 0.2) (layer "F.Cu") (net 9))
 (segment (start 141.92331 121.04) (end 153.12 121.04) (width 0.2) (layer "F.Cu") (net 9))
 (segment (start 154.183 98.470684) (end 154.183 117.437) (width 0.2) (layer "B.Cu") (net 10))
 (segment (start 154.183 117.437) (end 153.12 118.5) (width 0.2) (layer "B.Cu") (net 10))
 (segment (start 141.44625 85.733934) (end 154.183 98.470684) (width 0.2) (layer "B.Cu") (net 10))
 (segment (start 141.44625 71.27875) (end 141.44625 85.733934) (width 0.2) (layer "B.Cu") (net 10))
 (segment (start 152.057 114.897) (end 153.12 115.96) (width 0.2) (layer "B.Cu") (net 6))
 (segment (start 130.82875 90.32875) (end 152.057 111.557) (width 0.2) (layer "B.Cu") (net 6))
 (segment (start 152.057 111.557) (end 152.057 114.897) (width 0.2) (layer "B.Cu") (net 6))
 (segment (start 122.39625 90.32875) (end 130.82875 90.32875) (width 0.2) (layer "B.Cu") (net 6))
 (segment (start 160.49625 107.08044) (end 154.15669 113.42) (width 0.2) (layer "F.Cu") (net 11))
 (segment (start 160.49625 90.32875) (end 160.49625 107.08044) (width 0.2) (layer "F.Cu") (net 11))
 (segment (start 154.15669 113.42) (end 153.12 113.42) (width 0.2) (layer "F.Cu") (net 11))
 (segment (start 141.44625 90.32875) (end 141.44625 99.20625) (width 0.2) (layer "F.Cu") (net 7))
 (segment (start 141.44625 99.20625) (end 153.12 110.88) (width 0.2) (layer "F.Cu") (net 7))
 (segment (start 122.39625 71.27875) (end 122.39625 88.347436) (width 0.2) (layer "B.Cu") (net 2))
 (segment (start 137.88 107.92403) (end 137.88 110.88) (width 0.2) (layer "B.Cu") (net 2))
 (segment (start 122.39625 88.347436) (end 120.99525 89.748436) (width 0.2) (layer "B.Cu") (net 2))
 (segment (start 120.99525 89.748436) (end 120.99525 91.03928) (width 0.2) (layer "B.Cu") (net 2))
 (segment (start 120.99525 91.03928) (end 137.88 107.92403) (width 0.2) (layer "B.Cu") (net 2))
 (segment (start 140.865936 88.92775) (end 138.943 90.850686) (width 0.2) (layer "F.Cu") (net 12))
 (segment (start 142.026564 88.92775) (end 140.865936 88.92775) (width 0.2) (layer "F.Cu") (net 12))
 (segment (start 160.49625 77.070064) (end 148.376564 89.18975) (width 0.2) (layer "F.Cu") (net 12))
 (segment (start 142.288564 89.18975) (end 142.026564 88.92775) (width 0.2) (layer "F.Cu") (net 12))
 (segment (start 148.376564 89.18975) (end 142.288564 89.18975) (width 0.2) (layer "F.Cu") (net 12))
 (segment (start 138.943 90.850686) (end 138.943 112.357) (width 0.2) (layer "F.Cu") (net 12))
 (segment (start 138.943 112.357) (end 137.88 113.42) (width 0.2) (layer "F.Cu") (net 12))
 (segment (start 160.49625 71.27875) (end 160.49625 77.070064) (width 0.2) (layer "F.Cu") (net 12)))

